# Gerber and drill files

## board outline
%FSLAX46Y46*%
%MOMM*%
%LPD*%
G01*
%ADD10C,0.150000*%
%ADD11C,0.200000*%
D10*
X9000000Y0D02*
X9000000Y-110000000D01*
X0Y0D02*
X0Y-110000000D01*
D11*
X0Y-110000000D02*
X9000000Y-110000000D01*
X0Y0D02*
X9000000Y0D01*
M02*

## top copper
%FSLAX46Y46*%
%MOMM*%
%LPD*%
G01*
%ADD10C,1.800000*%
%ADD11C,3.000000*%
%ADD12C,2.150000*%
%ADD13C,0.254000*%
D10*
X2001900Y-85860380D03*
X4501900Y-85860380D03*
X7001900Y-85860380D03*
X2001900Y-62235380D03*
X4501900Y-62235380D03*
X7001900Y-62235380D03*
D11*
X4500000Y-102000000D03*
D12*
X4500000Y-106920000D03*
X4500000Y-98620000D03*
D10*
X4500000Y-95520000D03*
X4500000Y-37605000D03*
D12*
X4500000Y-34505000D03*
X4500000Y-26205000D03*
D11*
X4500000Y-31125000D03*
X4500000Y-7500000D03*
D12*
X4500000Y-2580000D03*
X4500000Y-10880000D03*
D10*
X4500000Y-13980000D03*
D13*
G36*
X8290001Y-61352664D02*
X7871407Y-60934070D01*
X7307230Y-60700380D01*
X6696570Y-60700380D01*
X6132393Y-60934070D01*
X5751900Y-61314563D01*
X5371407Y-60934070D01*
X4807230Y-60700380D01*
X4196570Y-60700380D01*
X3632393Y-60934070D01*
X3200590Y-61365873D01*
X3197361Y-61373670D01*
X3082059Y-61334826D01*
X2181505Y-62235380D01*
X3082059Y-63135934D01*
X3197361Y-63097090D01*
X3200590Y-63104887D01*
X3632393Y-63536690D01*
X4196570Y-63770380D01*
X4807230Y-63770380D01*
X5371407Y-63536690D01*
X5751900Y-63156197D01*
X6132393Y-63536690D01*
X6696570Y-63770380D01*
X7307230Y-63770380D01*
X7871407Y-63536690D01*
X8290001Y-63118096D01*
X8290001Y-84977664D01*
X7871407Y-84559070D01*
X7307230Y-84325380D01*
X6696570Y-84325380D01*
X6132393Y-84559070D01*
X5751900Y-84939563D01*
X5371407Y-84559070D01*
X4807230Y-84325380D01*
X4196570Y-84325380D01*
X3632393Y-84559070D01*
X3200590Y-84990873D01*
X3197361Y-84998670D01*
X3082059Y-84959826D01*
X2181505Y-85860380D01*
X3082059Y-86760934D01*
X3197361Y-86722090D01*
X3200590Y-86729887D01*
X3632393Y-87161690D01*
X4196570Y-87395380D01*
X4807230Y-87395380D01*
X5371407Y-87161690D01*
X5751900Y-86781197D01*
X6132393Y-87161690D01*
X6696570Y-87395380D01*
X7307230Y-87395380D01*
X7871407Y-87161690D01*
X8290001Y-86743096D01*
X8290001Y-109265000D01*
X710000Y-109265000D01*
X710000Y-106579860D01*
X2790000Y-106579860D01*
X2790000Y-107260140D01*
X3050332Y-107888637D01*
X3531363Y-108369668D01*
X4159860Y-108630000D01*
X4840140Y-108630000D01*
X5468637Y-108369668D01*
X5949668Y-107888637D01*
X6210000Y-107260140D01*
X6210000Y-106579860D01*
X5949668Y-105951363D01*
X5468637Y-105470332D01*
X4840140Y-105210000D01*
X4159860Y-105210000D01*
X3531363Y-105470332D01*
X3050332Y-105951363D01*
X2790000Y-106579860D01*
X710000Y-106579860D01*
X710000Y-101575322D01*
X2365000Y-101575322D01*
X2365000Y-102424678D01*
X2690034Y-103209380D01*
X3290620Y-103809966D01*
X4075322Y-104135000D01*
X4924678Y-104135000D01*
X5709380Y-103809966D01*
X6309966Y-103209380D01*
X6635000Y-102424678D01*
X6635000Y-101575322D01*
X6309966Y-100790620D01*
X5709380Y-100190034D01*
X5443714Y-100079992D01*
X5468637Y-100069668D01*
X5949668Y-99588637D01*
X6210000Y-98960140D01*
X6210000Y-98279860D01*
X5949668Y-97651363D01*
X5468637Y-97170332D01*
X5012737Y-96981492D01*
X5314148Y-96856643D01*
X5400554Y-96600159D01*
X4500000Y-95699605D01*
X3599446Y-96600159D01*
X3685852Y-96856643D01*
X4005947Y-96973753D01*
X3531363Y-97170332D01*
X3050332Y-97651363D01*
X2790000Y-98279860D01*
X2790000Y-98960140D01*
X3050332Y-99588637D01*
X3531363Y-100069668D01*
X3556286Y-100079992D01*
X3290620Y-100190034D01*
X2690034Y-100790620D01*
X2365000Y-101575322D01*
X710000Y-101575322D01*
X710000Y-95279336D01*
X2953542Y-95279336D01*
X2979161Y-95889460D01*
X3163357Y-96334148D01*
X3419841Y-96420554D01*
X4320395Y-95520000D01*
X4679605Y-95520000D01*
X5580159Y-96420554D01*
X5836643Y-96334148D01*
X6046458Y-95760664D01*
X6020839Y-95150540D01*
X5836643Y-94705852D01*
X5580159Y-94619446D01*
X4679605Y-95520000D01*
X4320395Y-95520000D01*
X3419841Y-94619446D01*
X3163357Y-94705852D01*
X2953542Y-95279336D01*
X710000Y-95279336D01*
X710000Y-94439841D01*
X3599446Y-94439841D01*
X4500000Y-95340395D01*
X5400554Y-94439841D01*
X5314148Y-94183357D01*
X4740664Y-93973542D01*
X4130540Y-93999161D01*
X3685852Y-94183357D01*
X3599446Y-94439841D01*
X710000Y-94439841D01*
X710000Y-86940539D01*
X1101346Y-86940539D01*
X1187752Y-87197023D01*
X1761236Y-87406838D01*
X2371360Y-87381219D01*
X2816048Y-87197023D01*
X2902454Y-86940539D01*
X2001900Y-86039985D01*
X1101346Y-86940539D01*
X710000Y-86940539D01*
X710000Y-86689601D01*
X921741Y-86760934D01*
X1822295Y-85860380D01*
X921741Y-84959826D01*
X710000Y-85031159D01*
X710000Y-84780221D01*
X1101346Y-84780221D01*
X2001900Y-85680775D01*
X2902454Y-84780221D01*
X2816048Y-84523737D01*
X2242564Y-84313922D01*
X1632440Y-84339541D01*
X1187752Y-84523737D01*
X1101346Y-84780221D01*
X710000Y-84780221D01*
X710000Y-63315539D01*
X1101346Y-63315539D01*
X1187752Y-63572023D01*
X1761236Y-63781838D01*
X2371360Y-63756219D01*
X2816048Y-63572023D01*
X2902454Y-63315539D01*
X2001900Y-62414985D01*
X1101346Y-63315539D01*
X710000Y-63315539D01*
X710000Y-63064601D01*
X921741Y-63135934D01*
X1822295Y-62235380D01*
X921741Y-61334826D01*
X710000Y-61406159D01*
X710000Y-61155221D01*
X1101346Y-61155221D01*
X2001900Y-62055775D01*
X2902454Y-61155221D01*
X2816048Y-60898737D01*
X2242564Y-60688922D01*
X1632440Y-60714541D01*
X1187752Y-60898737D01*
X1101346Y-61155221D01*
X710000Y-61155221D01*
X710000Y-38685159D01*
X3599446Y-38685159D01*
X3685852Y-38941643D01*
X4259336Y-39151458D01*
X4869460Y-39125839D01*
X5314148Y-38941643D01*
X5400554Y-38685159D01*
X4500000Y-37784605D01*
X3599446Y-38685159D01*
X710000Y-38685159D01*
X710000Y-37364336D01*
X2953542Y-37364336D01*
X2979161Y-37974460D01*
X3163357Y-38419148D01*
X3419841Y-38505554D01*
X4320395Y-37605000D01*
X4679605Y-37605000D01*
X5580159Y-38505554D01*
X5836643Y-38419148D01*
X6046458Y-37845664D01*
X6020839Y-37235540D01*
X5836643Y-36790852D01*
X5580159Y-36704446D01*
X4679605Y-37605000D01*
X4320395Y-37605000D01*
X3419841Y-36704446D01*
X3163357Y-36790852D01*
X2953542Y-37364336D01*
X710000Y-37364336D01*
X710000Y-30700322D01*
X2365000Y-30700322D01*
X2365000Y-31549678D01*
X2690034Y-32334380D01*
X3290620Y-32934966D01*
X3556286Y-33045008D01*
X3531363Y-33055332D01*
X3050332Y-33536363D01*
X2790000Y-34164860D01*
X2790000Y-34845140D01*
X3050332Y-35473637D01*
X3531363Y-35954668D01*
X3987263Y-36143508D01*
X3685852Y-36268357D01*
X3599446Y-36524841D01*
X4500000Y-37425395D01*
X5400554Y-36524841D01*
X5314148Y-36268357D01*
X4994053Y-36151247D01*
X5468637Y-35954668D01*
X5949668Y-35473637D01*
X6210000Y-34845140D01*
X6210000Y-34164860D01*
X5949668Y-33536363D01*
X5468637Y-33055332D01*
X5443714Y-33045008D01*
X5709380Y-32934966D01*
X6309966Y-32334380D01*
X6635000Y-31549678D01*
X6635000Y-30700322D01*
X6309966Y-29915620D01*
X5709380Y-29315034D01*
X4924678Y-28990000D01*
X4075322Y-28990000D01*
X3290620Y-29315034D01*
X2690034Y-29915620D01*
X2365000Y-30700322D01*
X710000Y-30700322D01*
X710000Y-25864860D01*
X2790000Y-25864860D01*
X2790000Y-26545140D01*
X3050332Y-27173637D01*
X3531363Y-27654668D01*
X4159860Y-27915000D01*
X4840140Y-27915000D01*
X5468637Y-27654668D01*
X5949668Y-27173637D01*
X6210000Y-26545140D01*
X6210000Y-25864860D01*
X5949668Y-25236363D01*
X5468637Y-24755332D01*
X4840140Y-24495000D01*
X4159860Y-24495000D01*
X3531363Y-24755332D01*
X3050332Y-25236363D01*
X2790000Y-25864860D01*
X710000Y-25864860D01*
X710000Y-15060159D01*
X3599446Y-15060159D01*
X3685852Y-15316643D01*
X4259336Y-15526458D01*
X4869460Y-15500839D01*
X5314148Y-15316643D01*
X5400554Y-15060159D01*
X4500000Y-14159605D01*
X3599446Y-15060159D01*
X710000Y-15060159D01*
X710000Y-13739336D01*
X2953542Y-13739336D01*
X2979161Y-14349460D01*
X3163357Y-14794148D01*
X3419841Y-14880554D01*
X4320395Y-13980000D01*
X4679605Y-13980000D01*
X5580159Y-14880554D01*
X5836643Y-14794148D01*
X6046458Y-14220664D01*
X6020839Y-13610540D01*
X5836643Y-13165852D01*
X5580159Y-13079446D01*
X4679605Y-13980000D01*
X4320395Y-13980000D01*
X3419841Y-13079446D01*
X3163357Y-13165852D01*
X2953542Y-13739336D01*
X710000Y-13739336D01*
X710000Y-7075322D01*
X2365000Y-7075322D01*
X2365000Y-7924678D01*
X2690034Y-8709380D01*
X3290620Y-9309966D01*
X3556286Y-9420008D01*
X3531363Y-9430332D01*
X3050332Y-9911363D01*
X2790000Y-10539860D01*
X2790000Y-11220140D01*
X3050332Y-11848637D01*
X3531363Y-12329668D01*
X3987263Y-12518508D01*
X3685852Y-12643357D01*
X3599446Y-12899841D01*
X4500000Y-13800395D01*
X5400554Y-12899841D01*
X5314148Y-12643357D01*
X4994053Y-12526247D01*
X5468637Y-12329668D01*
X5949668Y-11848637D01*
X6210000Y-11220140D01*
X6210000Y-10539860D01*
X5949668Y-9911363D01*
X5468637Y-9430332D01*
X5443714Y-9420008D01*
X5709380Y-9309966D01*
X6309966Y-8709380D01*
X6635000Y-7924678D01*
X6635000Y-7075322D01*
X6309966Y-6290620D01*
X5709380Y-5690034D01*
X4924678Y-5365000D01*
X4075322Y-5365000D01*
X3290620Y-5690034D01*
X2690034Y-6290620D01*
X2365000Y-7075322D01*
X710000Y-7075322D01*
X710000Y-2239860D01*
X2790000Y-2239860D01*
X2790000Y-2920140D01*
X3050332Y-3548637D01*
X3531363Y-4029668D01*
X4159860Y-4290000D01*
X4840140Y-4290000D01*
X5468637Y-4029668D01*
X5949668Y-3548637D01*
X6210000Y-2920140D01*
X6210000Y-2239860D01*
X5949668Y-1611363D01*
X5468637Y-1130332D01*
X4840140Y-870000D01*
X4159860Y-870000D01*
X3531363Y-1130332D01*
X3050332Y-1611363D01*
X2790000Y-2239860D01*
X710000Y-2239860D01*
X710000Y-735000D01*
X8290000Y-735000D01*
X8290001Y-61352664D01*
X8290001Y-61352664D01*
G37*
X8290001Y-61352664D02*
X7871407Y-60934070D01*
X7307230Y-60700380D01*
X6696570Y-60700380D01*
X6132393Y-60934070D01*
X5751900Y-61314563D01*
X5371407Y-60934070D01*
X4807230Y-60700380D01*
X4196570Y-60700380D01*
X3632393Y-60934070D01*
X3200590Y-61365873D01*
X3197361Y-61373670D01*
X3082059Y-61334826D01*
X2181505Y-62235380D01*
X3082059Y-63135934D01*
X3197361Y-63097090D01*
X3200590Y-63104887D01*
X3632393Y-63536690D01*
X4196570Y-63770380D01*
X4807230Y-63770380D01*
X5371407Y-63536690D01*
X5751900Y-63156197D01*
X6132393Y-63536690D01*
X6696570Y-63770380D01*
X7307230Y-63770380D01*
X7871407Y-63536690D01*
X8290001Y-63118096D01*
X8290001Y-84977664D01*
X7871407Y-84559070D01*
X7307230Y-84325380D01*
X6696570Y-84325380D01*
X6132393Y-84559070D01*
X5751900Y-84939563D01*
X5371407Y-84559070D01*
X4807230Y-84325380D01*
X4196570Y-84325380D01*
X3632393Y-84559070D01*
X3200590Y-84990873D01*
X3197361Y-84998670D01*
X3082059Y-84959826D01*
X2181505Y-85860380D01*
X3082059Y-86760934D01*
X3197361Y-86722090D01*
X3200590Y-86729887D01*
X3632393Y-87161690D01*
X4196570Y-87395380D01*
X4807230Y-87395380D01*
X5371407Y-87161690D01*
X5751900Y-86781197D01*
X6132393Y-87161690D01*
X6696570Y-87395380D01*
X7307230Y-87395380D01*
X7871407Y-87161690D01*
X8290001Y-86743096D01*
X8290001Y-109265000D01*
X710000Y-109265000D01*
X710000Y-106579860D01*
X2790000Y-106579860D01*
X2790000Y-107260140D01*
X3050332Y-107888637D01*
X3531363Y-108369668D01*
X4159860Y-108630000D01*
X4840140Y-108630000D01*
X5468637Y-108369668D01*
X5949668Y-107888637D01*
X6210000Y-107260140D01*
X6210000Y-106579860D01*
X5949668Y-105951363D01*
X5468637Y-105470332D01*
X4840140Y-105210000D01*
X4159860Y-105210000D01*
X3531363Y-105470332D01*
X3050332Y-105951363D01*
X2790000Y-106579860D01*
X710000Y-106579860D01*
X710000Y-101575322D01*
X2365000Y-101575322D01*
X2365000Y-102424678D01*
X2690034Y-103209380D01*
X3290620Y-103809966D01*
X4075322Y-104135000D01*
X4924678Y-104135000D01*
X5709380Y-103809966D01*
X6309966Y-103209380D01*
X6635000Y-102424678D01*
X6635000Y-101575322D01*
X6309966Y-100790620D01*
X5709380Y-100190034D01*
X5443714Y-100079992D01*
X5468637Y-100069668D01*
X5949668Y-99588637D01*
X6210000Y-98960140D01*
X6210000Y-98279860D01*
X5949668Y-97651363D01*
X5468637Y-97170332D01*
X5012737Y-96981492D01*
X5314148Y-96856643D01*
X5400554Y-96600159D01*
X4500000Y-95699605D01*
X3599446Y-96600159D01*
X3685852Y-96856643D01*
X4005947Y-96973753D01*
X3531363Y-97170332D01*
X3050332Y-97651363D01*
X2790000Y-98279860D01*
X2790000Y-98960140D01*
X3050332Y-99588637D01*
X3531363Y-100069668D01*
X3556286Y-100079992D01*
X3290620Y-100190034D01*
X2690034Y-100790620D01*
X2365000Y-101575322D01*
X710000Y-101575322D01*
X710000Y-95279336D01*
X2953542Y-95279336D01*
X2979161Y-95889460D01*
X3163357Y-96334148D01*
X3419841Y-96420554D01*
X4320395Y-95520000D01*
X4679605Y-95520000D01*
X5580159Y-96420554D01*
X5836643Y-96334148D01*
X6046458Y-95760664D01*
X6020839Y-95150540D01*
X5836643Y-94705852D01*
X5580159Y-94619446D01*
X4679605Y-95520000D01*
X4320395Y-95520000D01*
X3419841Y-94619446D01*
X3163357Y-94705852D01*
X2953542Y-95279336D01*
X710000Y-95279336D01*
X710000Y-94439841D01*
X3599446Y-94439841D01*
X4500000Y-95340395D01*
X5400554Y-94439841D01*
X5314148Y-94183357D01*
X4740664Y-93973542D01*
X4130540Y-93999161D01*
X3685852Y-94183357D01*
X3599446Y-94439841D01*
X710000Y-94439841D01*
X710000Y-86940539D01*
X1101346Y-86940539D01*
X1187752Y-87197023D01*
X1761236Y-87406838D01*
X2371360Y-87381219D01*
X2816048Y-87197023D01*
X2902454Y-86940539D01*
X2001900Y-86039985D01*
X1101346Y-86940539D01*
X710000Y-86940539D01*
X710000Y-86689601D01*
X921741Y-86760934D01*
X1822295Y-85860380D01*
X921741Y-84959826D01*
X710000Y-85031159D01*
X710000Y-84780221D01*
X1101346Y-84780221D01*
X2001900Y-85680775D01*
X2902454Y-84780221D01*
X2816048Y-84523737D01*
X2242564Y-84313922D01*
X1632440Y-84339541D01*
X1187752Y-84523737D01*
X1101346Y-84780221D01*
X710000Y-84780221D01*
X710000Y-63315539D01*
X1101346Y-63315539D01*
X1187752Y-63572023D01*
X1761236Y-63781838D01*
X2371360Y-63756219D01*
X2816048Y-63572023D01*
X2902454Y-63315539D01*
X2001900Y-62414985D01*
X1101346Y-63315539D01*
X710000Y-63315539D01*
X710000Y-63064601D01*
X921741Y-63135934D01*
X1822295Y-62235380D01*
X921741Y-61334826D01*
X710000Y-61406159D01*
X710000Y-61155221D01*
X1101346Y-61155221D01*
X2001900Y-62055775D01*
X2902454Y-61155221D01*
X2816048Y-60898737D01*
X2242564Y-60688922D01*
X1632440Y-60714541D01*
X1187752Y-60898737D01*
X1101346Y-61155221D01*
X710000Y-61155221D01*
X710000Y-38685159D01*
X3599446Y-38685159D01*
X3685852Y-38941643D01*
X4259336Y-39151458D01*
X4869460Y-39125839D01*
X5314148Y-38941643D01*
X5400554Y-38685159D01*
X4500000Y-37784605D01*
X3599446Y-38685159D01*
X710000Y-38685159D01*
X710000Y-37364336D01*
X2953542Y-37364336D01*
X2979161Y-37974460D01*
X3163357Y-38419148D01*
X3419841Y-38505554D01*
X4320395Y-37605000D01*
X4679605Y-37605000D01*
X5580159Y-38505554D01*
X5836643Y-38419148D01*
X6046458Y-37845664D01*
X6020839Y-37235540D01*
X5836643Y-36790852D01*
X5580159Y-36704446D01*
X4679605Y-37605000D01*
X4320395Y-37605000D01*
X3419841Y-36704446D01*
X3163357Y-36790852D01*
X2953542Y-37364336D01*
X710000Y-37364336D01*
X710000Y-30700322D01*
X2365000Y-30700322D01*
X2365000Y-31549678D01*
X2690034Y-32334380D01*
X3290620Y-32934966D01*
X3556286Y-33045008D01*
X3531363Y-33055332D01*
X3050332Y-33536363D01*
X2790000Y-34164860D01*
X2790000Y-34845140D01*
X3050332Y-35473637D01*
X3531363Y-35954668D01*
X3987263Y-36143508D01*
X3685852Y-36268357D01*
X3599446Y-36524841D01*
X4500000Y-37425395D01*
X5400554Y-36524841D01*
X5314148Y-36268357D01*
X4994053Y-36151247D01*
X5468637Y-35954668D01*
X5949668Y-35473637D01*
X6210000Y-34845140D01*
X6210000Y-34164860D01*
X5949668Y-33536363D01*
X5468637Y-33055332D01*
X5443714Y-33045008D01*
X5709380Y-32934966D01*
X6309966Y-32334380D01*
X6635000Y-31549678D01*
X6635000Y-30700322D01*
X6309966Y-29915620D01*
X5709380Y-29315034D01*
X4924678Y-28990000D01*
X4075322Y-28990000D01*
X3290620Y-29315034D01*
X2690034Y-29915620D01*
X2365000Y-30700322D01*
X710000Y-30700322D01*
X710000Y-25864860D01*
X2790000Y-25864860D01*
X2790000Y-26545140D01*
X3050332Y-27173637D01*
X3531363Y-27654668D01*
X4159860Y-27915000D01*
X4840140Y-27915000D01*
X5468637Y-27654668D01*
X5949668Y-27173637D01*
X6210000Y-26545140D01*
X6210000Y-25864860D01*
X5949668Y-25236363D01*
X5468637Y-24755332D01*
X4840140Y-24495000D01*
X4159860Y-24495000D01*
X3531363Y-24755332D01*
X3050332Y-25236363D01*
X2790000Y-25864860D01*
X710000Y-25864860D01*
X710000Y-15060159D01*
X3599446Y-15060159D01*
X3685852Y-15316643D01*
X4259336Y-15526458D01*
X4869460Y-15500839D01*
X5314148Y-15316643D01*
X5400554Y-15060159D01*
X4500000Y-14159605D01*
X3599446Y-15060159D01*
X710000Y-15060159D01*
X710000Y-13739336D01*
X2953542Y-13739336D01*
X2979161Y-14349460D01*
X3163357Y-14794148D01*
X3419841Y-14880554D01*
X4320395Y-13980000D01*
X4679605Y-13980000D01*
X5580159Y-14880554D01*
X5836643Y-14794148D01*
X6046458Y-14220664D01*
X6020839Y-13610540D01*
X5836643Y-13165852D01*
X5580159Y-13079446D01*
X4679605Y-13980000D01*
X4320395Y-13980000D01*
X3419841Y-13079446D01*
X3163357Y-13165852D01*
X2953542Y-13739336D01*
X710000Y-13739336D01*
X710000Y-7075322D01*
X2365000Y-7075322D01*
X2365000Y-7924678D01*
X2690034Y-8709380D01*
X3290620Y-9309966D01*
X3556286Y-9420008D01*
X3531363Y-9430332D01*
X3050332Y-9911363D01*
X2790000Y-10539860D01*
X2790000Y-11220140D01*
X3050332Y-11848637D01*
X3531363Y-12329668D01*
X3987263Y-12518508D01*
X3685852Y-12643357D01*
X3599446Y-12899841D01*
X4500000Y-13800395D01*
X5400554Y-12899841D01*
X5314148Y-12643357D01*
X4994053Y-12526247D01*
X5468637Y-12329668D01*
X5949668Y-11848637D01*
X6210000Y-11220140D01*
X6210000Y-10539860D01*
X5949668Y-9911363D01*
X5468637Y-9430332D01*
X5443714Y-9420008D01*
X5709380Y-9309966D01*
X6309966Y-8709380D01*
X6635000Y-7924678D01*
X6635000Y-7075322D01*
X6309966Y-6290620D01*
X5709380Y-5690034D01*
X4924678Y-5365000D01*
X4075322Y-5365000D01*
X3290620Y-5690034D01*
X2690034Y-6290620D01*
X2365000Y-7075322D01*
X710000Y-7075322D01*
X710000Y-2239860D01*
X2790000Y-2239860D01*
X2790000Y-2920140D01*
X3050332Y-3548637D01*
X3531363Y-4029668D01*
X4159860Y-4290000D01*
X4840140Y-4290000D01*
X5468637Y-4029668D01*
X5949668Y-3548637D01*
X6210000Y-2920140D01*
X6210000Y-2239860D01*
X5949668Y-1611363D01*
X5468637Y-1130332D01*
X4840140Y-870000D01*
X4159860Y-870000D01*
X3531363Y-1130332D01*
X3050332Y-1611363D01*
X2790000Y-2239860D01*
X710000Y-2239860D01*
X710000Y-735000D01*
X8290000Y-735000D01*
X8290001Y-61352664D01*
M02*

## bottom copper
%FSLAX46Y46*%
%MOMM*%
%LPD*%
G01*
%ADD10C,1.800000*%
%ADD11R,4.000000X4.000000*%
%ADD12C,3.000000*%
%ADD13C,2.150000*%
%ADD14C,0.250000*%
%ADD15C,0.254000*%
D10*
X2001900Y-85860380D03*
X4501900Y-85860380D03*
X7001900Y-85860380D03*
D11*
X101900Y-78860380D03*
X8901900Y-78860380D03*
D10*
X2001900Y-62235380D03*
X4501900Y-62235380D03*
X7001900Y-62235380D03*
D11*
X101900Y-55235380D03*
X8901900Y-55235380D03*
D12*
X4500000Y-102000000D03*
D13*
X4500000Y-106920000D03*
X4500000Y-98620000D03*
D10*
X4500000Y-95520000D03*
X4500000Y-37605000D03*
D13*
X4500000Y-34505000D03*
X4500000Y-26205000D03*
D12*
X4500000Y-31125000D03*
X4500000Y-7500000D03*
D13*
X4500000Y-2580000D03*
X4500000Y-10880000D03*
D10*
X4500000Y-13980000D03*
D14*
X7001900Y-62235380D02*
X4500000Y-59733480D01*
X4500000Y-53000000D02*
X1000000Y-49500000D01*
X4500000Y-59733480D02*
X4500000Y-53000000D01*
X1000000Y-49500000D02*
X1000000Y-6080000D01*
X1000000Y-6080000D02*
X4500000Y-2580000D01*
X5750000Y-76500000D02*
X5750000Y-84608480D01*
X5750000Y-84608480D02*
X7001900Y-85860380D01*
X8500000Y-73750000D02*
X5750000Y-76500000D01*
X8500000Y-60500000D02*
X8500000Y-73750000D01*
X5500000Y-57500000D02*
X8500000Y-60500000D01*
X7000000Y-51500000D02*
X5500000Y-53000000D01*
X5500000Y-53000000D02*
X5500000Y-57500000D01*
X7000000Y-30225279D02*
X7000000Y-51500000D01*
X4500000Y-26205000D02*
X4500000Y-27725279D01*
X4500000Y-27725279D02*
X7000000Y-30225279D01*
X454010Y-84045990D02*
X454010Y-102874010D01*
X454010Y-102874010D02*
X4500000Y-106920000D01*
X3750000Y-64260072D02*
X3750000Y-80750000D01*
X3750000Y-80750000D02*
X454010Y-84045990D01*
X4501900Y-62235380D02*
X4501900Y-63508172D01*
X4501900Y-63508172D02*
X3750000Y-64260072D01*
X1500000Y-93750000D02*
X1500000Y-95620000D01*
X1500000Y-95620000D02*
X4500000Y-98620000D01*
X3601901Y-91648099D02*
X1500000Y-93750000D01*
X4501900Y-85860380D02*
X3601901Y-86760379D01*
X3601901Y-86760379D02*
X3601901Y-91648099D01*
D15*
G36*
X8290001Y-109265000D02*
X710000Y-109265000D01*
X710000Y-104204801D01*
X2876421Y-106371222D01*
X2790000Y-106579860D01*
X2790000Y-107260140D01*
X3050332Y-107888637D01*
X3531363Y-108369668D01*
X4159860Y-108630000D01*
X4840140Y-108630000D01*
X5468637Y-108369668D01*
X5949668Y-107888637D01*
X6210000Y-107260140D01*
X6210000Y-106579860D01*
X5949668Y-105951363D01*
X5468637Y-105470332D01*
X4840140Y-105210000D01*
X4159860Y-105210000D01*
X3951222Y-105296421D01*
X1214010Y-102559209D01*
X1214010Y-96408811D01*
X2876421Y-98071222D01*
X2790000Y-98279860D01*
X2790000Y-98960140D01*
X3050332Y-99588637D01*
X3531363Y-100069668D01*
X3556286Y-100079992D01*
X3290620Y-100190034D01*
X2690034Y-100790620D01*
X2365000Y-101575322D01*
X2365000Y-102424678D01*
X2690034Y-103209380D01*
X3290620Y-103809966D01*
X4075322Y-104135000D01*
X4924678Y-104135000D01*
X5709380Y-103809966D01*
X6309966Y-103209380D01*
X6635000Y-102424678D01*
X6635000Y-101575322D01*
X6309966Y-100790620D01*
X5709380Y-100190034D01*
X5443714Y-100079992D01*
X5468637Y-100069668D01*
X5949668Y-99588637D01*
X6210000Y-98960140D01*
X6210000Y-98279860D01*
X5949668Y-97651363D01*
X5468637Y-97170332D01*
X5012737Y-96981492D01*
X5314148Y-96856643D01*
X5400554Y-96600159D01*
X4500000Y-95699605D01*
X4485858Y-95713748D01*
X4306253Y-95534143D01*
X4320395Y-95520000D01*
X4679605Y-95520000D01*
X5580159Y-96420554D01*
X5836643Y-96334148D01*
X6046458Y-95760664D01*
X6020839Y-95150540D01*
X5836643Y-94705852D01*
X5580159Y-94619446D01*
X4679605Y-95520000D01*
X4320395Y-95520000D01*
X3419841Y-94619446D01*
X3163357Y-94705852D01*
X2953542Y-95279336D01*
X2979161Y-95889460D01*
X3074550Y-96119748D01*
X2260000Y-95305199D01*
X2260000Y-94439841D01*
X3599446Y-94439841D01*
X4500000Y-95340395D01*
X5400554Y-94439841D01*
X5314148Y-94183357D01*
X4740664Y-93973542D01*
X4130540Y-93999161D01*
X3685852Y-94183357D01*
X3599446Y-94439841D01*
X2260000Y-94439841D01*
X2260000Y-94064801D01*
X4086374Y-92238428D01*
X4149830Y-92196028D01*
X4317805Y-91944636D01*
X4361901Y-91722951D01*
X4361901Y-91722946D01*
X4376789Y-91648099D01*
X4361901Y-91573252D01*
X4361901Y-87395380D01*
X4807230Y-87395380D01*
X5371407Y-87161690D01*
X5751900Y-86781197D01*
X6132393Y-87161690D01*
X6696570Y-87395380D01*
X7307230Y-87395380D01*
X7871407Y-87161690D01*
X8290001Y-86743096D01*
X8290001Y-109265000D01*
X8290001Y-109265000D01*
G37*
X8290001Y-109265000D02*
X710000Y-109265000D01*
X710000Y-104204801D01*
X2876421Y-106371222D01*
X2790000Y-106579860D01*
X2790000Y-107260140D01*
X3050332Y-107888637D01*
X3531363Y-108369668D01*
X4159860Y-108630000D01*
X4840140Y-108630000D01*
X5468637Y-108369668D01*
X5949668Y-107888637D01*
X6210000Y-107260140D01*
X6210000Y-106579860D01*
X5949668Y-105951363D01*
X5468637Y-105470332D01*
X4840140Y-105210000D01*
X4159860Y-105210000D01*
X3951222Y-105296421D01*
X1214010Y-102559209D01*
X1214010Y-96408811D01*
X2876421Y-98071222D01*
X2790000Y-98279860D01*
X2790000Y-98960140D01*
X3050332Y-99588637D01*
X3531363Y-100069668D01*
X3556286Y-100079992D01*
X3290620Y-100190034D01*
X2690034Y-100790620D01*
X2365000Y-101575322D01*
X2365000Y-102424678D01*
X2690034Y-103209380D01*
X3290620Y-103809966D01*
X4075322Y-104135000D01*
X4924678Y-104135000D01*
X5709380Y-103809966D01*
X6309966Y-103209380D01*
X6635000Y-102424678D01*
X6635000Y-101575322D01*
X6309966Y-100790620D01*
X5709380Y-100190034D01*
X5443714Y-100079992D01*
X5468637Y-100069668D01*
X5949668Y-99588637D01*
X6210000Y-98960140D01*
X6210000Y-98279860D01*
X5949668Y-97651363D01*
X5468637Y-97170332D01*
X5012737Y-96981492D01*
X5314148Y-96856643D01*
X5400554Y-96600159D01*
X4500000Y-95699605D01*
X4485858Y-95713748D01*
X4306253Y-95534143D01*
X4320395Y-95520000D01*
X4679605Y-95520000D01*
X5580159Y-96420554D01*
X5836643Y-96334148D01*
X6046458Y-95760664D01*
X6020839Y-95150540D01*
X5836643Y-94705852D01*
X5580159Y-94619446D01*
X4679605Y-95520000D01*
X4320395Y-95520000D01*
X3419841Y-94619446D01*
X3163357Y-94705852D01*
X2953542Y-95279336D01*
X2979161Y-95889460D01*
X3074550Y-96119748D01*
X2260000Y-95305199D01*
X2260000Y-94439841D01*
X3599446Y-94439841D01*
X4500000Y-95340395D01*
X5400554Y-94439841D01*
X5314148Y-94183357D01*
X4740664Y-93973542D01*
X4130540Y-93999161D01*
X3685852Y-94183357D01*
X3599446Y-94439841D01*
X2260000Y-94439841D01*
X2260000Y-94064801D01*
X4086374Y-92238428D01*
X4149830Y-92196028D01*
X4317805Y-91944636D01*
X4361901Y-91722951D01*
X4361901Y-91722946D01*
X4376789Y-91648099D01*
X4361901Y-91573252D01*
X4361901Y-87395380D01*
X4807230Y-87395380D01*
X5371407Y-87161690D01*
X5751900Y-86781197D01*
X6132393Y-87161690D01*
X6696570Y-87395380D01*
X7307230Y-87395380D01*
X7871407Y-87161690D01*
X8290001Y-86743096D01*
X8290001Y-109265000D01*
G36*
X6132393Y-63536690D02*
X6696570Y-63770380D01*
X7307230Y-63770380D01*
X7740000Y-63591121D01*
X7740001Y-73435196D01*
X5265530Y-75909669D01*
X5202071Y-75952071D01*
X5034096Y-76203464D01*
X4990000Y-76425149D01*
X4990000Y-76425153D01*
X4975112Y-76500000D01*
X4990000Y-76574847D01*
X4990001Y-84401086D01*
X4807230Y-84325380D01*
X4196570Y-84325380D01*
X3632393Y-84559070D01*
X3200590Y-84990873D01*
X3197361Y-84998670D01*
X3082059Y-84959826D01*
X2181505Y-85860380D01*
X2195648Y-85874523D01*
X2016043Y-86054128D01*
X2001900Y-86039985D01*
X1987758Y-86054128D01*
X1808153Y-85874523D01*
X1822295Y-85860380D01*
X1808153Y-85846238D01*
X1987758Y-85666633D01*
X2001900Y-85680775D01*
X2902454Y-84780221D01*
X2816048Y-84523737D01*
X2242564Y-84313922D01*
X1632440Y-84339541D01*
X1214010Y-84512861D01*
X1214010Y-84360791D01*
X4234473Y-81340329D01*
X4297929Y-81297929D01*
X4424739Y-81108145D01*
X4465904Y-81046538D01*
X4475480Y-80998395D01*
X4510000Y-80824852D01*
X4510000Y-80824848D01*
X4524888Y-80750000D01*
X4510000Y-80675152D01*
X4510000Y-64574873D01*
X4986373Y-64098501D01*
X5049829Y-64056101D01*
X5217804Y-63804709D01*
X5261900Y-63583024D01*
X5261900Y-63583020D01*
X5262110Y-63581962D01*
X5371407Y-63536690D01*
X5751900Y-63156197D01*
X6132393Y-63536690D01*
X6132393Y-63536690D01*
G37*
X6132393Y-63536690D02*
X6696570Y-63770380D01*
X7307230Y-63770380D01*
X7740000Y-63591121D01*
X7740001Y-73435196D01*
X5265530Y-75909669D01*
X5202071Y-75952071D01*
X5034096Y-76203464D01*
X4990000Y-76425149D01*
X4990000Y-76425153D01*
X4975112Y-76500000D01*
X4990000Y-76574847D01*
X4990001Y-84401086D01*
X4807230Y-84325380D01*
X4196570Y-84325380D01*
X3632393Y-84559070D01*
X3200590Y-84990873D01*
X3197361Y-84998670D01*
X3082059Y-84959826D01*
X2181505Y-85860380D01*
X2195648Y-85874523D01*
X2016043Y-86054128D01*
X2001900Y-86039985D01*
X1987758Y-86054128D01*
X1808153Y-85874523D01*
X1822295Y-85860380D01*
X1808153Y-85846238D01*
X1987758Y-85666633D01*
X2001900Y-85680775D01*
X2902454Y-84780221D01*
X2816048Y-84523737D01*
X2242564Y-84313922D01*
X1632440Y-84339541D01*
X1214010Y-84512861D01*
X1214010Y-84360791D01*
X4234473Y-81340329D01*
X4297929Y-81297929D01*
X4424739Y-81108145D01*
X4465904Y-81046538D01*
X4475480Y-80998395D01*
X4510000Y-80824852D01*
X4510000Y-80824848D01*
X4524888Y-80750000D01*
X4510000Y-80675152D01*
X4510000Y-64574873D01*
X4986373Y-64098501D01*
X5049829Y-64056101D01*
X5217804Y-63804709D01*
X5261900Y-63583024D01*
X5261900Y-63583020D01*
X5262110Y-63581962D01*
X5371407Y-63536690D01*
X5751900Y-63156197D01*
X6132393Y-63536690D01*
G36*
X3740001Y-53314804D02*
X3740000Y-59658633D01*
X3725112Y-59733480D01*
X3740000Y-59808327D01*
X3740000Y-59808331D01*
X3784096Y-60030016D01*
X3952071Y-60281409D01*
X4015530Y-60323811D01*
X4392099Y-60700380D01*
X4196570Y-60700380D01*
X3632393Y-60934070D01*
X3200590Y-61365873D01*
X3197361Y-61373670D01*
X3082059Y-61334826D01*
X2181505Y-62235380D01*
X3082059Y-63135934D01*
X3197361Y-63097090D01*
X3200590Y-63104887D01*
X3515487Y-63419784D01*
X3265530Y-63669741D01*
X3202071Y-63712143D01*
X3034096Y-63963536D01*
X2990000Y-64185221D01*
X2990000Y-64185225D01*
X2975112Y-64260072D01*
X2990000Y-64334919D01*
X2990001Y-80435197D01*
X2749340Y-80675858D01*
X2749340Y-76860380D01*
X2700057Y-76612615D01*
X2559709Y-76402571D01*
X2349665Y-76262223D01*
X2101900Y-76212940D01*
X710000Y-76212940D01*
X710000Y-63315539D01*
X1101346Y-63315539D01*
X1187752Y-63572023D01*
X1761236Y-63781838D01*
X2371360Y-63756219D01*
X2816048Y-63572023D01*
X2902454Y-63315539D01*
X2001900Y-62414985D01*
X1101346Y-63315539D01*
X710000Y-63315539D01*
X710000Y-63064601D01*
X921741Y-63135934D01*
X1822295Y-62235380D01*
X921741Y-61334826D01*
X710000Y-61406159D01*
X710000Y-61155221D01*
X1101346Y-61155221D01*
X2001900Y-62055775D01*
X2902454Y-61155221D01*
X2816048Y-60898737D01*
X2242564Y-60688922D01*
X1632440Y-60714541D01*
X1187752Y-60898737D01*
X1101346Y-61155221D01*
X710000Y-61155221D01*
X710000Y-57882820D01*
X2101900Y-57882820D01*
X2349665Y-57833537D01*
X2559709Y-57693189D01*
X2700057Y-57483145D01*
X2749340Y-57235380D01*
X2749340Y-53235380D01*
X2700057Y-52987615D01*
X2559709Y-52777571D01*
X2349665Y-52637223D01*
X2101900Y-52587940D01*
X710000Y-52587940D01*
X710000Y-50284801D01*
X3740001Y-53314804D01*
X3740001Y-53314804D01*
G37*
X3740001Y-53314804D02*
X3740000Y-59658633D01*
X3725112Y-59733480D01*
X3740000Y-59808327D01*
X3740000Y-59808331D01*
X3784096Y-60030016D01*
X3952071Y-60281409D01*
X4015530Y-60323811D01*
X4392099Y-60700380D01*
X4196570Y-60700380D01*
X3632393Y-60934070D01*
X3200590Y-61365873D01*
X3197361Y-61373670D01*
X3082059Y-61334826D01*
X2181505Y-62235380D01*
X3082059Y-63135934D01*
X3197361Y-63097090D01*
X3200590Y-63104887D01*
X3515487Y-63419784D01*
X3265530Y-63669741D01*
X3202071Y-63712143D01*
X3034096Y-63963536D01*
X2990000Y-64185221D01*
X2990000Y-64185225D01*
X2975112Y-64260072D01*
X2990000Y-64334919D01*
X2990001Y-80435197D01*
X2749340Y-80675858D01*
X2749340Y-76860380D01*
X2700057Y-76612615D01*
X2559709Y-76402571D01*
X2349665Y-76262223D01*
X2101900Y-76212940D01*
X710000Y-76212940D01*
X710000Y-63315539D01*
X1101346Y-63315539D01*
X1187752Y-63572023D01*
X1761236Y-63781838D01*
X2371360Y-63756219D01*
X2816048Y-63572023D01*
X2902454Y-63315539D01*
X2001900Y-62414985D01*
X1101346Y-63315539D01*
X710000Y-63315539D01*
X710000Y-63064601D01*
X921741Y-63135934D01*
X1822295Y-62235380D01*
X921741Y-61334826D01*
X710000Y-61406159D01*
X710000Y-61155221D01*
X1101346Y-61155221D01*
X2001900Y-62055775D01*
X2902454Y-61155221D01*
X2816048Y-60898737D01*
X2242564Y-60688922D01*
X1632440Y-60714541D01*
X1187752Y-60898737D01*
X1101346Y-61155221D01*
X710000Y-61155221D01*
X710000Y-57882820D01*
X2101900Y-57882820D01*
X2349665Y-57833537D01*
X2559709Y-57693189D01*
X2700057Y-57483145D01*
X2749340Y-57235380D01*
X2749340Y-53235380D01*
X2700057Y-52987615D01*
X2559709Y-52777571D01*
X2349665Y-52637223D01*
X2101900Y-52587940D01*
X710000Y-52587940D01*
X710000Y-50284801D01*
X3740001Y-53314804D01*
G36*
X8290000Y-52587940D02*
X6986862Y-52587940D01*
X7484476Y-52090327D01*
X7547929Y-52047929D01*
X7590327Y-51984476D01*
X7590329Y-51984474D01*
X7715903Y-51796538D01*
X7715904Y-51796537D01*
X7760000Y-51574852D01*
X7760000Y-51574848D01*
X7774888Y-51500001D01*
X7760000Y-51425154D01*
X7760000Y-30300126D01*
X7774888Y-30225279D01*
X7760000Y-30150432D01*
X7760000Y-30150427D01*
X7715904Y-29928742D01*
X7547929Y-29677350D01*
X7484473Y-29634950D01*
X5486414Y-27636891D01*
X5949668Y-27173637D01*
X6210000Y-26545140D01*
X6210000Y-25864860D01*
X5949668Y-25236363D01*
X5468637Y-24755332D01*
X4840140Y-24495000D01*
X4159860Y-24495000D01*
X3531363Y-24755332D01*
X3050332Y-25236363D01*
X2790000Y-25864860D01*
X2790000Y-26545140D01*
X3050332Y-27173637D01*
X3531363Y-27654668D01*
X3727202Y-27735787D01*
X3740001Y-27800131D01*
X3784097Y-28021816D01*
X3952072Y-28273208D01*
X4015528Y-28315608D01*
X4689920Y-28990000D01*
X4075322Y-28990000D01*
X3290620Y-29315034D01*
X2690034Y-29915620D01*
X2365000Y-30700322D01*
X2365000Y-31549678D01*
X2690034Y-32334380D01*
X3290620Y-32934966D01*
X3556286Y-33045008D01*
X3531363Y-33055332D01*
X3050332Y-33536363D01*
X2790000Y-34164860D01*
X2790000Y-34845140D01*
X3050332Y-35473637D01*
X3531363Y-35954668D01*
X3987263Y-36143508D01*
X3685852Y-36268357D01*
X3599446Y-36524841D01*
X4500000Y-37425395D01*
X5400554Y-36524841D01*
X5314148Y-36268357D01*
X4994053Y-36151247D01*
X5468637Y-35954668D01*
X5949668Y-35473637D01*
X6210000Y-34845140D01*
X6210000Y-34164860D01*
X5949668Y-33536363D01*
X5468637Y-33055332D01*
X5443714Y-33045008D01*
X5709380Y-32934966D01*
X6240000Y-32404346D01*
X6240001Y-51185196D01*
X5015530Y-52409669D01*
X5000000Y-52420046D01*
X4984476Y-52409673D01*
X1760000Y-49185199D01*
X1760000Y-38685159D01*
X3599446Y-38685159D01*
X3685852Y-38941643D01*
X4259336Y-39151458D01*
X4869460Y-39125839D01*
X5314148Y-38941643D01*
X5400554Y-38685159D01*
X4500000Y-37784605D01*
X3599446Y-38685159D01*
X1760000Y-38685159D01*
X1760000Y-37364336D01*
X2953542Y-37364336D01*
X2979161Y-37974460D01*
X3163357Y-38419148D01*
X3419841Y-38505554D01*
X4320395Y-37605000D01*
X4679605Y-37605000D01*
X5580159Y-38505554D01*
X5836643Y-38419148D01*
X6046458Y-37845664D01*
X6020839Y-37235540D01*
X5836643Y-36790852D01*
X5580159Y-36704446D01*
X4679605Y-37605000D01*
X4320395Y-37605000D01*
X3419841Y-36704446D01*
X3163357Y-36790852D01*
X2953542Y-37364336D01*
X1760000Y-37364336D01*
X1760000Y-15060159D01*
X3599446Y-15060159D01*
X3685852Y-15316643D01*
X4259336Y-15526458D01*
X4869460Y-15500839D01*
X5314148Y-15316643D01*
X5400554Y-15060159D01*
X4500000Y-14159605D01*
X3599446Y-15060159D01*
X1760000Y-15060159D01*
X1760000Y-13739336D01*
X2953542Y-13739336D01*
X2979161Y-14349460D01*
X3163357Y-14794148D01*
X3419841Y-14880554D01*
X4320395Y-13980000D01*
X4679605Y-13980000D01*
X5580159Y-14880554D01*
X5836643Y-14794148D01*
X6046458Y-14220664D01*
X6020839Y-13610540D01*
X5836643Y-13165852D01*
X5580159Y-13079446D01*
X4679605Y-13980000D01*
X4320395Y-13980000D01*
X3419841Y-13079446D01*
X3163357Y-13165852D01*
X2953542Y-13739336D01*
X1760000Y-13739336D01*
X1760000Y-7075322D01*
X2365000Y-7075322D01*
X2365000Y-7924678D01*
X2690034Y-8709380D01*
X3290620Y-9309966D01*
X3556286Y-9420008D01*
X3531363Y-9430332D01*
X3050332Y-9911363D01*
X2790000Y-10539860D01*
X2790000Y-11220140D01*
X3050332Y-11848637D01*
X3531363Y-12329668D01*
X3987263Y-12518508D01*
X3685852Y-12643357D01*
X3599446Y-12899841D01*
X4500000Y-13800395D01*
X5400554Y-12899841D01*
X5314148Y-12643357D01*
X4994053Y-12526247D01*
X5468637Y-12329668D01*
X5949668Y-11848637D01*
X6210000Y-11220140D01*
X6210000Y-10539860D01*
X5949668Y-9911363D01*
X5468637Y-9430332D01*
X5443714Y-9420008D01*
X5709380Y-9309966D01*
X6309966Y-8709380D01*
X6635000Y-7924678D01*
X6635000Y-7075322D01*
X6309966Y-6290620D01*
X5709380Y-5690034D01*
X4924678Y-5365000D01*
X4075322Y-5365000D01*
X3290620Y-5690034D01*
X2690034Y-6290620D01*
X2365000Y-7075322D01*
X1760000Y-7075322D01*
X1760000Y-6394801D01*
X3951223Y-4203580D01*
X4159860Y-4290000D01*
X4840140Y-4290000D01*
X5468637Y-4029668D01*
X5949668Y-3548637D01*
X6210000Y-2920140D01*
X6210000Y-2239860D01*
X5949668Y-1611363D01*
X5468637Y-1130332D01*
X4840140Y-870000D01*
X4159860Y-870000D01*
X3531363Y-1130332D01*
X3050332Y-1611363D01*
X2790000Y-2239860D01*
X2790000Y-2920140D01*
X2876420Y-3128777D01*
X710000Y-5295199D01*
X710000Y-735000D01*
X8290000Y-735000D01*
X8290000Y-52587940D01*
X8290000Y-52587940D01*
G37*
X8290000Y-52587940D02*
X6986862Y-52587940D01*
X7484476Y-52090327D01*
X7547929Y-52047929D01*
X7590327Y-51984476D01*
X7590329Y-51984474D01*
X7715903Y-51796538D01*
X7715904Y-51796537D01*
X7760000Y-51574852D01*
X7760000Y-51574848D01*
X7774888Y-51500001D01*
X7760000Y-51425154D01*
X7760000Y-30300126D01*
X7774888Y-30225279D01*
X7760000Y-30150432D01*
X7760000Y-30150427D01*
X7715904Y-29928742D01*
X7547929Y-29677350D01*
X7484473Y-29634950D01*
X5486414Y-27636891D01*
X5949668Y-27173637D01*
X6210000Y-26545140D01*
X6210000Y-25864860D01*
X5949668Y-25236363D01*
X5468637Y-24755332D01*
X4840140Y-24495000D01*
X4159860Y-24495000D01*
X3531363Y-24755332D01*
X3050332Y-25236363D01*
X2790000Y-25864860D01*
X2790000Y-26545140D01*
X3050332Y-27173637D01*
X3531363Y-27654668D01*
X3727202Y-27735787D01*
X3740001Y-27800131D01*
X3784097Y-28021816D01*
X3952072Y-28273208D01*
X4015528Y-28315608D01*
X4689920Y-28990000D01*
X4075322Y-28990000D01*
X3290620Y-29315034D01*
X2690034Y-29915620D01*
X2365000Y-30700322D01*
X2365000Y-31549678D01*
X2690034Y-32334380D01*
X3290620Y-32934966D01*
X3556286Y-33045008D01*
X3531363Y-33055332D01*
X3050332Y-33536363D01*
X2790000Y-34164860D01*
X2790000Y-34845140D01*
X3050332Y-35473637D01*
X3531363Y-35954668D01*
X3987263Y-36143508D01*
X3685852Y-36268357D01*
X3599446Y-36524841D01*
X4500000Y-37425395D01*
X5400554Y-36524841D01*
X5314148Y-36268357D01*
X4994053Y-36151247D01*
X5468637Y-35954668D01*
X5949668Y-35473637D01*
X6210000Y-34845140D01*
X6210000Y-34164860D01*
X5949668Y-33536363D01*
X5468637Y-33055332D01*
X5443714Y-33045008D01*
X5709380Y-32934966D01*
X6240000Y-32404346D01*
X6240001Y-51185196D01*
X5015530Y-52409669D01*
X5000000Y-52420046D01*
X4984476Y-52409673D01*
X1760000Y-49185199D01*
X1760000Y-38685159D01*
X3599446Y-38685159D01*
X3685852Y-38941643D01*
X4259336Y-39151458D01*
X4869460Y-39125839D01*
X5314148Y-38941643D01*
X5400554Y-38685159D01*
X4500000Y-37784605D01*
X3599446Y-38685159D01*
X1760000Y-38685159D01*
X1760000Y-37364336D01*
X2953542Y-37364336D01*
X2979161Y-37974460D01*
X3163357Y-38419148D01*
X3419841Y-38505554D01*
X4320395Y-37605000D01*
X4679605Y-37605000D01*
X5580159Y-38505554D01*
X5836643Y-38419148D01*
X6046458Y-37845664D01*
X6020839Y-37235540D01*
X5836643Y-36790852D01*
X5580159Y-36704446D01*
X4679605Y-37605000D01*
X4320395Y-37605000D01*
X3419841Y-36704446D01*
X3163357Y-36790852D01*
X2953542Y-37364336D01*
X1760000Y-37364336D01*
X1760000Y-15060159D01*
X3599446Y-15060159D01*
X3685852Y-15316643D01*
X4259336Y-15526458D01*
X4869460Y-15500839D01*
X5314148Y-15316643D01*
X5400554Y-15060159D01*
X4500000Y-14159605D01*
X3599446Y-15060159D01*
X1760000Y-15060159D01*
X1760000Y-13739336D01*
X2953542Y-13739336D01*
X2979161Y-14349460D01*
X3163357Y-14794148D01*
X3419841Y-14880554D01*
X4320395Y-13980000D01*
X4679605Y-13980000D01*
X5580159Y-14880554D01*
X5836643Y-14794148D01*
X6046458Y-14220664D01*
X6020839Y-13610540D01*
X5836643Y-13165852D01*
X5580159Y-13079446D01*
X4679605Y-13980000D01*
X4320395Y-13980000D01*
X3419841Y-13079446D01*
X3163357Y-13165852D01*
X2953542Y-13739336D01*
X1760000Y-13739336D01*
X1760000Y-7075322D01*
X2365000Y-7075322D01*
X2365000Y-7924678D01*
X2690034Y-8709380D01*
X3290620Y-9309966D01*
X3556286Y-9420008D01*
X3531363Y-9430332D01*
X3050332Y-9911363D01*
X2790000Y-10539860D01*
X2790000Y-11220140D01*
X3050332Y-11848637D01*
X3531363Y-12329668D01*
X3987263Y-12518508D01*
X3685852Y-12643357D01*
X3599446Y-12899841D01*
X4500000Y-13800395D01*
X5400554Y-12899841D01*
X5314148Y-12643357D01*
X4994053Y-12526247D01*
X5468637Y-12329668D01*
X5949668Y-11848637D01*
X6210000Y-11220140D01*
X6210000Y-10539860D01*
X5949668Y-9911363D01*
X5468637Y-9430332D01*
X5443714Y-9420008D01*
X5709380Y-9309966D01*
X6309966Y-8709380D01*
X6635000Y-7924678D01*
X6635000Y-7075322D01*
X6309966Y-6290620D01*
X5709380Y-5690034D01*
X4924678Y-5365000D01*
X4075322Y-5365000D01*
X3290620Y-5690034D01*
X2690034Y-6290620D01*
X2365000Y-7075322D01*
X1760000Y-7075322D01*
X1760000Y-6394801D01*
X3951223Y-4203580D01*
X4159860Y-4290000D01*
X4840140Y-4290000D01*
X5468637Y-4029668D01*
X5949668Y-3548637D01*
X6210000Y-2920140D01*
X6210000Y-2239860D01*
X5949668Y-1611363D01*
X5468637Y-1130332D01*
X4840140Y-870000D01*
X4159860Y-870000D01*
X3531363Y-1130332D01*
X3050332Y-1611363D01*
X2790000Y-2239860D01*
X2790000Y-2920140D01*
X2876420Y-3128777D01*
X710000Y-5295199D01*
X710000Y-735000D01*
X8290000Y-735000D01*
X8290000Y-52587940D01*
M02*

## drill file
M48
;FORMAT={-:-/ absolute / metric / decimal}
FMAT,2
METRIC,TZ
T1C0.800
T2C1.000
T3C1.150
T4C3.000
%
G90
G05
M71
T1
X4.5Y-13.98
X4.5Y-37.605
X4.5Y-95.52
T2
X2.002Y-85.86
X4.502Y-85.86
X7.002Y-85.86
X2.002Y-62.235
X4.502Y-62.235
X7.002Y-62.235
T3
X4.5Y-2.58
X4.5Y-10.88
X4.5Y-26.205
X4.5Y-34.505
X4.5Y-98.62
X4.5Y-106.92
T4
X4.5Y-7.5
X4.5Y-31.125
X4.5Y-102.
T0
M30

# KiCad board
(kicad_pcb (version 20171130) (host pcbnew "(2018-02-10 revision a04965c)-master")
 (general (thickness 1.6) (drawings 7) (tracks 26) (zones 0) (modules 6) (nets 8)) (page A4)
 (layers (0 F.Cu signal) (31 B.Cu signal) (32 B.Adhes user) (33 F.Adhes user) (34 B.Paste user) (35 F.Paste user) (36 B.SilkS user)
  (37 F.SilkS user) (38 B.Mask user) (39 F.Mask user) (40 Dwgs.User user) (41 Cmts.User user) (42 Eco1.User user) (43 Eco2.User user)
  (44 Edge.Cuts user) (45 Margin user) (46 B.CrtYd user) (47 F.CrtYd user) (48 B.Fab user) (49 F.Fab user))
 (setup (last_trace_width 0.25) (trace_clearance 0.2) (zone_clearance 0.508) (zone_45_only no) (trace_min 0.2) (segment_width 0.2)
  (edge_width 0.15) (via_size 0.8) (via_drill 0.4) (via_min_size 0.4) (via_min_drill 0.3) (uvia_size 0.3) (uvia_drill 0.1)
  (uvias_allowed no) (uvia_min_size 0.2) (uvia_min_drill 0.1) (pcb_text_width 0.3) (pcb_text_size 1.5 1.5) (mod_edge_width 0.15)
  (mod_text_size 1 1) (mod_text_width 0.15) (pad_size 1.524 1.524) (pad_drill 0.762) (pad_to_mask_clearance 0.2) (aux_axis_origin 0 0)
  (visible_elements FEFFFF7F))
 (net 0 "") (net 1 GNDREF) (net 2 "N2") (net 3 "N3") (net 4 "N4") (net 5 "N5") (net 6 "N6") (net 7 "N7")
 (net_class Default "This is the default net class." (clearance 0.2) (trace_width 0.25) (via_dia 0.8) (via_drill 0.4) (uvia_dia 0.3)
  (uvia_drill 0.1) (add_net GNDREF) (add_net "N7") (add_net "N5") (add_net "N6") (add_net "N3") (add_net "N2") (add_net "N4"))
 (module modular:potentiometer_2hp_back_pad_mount (layer F.Cu) (at 4.5 78.375 90)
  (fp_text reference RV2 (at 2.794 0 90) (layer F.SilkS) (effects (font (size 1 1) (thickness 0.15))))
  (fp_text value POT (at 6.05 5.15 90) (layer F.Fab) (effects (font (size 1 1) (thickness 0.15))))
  (pad 1 thru_hole circle (at -7.48538 -2.4981 90) (size 1.8 1.8) (drill 1) (layers *.Cu *.Mask) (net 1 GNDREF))
  (pad 2 thru_hole circle (at -7.48538 0.0019 90) (size 1.8 1.8) (drill 1) (layers *.Cu *.Mask) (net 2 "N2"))
  (pad 3 thru_hole circle (at -7.48538 2.5019 90) (size 1.8 1.8) (drill 1) (layers *.Cu *.Mask) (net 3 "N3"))
  (pad 0 smd rect (at -0.48538 -4.3981 90) (size 4 4) (layers B.Cu B.Mask))
  (pad 0 smd rect (at -0.48538 4.4019 90) (size 4 4) (layers B.Cu B.Mask)))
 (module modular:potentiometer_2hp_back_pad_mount (layer F.Cu) (at 4.5 54.75 90)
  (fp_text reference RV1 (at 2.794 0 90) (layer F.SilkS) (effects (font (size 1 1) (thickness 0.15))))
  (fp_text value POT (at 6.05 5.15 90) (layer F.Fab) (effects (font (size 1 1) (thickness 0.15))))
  (pad 1 thru_hole circle (at -7.48538 -2.4981 90) (size 1.8 1.8) (drill 1) (layers *.Cu *.Mask) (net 1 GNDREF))
  (pad 2 thru_hole circle (at -7.48538 0.0019 90) (size 1.8 1.8) (drill 1) (layers *.Cu *.Mask) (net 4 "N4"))
  (pad 3 thru_hole circle (at -7.48538 2.5019 90) (size 1.8 1.8) (drill 1) (layers *.Cu *.Mask) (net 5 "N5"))
  (pad 0 smd rect (at -0.48538 -4.3981 90) (size 4 4) (layers B.Cu B.Mask))
  (pad 0 smd rect (at -0.48538 4.4019 90) (size 4 4) (layers B.Cu B.Mask)))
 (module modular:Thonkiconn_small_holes (layer F.Cu) (at 4.5 102 180)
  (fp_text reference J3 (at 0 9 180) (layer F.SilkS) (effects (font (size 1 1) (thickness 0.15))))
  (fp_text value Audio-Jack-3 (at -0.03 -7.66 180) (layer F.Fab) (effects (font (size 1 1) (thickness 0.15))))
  (pad "" thru_hole circle (at 0 0 180) (size 3 3) (drill 3) (layers *.Cu *.Mask F.SilkS))
  (pad 3 thru_hole circle (at 0 -4.92 180) (size 2.15 2.15) (drill 1.15) (layers *.Cu *.Mask F.SilkS) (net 4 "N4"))
  (pad 2 thru_hole circle (at 0 3.38 180) (size 2.15 2.15) (drill 1.15) (layers *.Cu *.Mask F.SilkS) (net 2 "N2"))
  (pad 1 thru_hole circle (at 0 6.48 180) (size 1.8 1.8) (drill 0.8) (layers *.Cu *.Mask F.SilkS) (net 1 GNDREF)))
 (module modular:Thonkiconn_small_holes (layer F.Cu) (at 4.5 31.125)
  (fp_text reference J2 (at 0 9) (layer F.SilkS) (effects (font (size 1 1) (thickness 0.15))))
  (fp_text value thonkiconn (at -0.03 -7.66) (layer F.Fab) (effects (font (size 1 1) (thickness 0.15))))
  (pad 1 thru_hole circle (at 0 6.48) (size 1.8 1.8) (drill 0.8) (layers *.Cu *.Mask F.SilkS) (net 1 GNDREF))
  (pad 2 thru_hole circle (at 0 3.38) (size 2.15 2.15) (drill 1.15) (layers *.Cu *.Mask F.SilkS) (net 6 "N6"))
  (pad 3 thru_hole circle (at 0 -4.92) (size 2.15 2.15) (drill 1.15) (layers *.Cu *.Mask F.SilkS) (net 3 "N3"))
  (pad "" thru_hole circle (at 0 0) (size 3 3) (drill 3) (layers *.Cu *.Mask F.SilkS)))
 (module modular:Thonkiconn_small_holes (layer F.Cu) (at 4.5 7.5)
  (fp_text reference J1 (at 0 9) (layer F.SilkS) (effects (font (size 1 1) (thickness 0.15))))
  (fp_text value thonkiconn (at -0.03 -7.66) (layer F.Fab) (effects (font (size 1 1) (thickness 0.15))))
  (pad "" thru_hole circle (at 0 0) (size 3 3) (drill 3) (layers *.Cu *.Mask F.SilkS))
  (pad 3 thru_hole circle (at 0 -4.92) (size 2.15 2.15) (drill 1.15) (layers *.Cu *.Mask F.SilkS) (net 5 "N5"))
  (pad 2 thru_hole circle (at 0 3.38) (size 2.15 2.15) (drill 1.15) (layers *.Cu *.Mask F.SilkS) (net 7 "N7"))
  (pad 1 thru_hole circle (at 0 6.48) (size 1.8 1.8) (drill 0.8) (layers *.Cu *.Mask F.SilkS) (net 1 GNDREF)))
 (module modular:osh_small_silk (layer B.Cu) (at 4.5 82.5 180)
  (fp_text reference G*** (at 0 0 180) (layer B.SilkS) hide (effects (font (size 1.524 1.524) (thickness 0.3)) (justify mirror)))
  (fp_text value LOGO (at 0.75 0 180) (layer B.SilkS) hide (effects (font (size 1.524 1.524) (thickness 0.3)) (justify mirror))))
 (gr_line (start 9 0) (end 9 110) (layer Edge.Cuts) (width 0.15))
 (gr_line (start 0 0) (end 0 110) (layer Edge.Cuts) (width 0.15))
 (gr_line (start 0 110) (end 9 110) (layer Edge.Cuts) (width 0.2))
 (gr_line (start 0 0) (end 9 0) (layer Edge.Cuts) (width 0.2))
 (segment (start 7.0019 62.23538) (end 4.5 59.73348) (width 0.25) (layer B.Cu) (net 5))
 (segment (start 4.5 53) (end 1 49.5) (width 0.25) (layer B.Cu) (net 5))
 (segment (start 4.5 59.73348) (end 4.5 53) (width 0.25) (layer B.Cu) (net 5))
 (segment (start 1 49.5) (end 1 6.08) (width 0.25) (layer B.Cu) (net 5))
 (segment (start 1 6.08) (end 4.5 2.58) (width 0.25) (layer B.Cu) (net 5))
 (segment (start 5.75 76.5) (end 5.75 84.60848) (width 0.25) (layer B.Cu) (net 3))
 (segment (start 5.75 84.60848) (end 7.0019 85.86038) (width 0.25) (layer B.Cu) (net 3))
 (segment (start 8.5 73.75) (end 5.75 76.5) (width 0.25) (layer B.Cu) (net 3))
 (segment (start 8.5 60.5) (end 8.5 73.75) (width 0.25) (layer B.Cu) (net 3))
 (segment (start 5.5 57.5) (end 8.5 60.5) (width 0.25) (layer B.Cu) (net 3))
 (segment (start 7 51.5) (end 5.5 53) (width 0.25) (layer B.Cu) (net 3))
 (segment (start 5.5 53) (end 5.5 57.5) (width 0.25) (layer B.Cu) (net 3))
 (segment (start 7 30.225279) (end 7 51.5) (width 0.25) (layer B.Cu) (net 3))
 (segment (start 4.5 26.205) (end 4.5 27.725279) (width 0.25) (layer B.Cu) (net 3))
 (segment (start 4.5 27.725279) (end 7 30.225279) (width 0.25) (layer B.Cu) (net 3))
 (segment (start 0.45401 84.04599) (end 0.45401 102.87401) (width 0.25) (layer B.Cu) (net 4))
 (segment (start 0.45401 102.87401) (end 4.5 106.92) (width 0.25) (layer B.Cu) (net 4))
 (segment (start 3.75 64.260072) (end 3.75 80.75) (width 0.25) (layer B.Cu) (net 4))
 (segment (start 3.75 80.75) (end 0.45401 84.04599) (width 0.25) (layer B.Cu) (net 4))
 (segment (start 4.5019 62.23538) (end 4.5019 63.508172) (width 0.25) (layer B.Cu) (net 4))
 (segment (start 4.5019 63.508172) (end 3.75 64.260072) (width 0.25) (layer B.Cu) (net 4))
 (segment (start 1.5 93.75) (end 1.5 95.62) (width 0.25) (layer B.Cu) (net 2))
 (segment (start 1.5 95.62) (end 4.5 98.62) (width 0.25) (layer B.Cu) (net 2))
 (segment (start 3.601901 91.648099) (end 1.5 93.75) (width 0.25) (layer B.Cu) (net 2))
 (segment (start 4.5019 85.86038) (end 3.601901 86.760379) (width 0.25) (layer B.Cu) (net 2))
 (segment (start 3.601901 86.760379) (end 3.601901 91.648099) (width 0.25) (layer B.Cu) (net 2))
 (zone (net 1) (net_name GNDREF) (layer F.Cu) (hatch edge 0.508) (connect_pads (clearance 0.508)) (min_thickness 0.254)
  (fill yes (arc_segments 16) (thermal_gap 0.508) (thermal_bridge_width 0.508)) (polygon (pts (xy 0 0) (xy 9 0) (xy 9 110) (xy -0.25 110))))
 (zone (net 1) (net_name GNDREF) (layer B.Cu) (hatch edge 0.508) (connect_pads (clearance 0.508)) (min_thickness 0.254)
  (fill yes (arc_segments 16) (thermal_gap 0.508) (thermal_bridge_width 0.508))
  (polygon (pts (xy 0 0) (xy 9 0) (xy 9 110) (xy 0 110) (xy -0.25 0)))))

